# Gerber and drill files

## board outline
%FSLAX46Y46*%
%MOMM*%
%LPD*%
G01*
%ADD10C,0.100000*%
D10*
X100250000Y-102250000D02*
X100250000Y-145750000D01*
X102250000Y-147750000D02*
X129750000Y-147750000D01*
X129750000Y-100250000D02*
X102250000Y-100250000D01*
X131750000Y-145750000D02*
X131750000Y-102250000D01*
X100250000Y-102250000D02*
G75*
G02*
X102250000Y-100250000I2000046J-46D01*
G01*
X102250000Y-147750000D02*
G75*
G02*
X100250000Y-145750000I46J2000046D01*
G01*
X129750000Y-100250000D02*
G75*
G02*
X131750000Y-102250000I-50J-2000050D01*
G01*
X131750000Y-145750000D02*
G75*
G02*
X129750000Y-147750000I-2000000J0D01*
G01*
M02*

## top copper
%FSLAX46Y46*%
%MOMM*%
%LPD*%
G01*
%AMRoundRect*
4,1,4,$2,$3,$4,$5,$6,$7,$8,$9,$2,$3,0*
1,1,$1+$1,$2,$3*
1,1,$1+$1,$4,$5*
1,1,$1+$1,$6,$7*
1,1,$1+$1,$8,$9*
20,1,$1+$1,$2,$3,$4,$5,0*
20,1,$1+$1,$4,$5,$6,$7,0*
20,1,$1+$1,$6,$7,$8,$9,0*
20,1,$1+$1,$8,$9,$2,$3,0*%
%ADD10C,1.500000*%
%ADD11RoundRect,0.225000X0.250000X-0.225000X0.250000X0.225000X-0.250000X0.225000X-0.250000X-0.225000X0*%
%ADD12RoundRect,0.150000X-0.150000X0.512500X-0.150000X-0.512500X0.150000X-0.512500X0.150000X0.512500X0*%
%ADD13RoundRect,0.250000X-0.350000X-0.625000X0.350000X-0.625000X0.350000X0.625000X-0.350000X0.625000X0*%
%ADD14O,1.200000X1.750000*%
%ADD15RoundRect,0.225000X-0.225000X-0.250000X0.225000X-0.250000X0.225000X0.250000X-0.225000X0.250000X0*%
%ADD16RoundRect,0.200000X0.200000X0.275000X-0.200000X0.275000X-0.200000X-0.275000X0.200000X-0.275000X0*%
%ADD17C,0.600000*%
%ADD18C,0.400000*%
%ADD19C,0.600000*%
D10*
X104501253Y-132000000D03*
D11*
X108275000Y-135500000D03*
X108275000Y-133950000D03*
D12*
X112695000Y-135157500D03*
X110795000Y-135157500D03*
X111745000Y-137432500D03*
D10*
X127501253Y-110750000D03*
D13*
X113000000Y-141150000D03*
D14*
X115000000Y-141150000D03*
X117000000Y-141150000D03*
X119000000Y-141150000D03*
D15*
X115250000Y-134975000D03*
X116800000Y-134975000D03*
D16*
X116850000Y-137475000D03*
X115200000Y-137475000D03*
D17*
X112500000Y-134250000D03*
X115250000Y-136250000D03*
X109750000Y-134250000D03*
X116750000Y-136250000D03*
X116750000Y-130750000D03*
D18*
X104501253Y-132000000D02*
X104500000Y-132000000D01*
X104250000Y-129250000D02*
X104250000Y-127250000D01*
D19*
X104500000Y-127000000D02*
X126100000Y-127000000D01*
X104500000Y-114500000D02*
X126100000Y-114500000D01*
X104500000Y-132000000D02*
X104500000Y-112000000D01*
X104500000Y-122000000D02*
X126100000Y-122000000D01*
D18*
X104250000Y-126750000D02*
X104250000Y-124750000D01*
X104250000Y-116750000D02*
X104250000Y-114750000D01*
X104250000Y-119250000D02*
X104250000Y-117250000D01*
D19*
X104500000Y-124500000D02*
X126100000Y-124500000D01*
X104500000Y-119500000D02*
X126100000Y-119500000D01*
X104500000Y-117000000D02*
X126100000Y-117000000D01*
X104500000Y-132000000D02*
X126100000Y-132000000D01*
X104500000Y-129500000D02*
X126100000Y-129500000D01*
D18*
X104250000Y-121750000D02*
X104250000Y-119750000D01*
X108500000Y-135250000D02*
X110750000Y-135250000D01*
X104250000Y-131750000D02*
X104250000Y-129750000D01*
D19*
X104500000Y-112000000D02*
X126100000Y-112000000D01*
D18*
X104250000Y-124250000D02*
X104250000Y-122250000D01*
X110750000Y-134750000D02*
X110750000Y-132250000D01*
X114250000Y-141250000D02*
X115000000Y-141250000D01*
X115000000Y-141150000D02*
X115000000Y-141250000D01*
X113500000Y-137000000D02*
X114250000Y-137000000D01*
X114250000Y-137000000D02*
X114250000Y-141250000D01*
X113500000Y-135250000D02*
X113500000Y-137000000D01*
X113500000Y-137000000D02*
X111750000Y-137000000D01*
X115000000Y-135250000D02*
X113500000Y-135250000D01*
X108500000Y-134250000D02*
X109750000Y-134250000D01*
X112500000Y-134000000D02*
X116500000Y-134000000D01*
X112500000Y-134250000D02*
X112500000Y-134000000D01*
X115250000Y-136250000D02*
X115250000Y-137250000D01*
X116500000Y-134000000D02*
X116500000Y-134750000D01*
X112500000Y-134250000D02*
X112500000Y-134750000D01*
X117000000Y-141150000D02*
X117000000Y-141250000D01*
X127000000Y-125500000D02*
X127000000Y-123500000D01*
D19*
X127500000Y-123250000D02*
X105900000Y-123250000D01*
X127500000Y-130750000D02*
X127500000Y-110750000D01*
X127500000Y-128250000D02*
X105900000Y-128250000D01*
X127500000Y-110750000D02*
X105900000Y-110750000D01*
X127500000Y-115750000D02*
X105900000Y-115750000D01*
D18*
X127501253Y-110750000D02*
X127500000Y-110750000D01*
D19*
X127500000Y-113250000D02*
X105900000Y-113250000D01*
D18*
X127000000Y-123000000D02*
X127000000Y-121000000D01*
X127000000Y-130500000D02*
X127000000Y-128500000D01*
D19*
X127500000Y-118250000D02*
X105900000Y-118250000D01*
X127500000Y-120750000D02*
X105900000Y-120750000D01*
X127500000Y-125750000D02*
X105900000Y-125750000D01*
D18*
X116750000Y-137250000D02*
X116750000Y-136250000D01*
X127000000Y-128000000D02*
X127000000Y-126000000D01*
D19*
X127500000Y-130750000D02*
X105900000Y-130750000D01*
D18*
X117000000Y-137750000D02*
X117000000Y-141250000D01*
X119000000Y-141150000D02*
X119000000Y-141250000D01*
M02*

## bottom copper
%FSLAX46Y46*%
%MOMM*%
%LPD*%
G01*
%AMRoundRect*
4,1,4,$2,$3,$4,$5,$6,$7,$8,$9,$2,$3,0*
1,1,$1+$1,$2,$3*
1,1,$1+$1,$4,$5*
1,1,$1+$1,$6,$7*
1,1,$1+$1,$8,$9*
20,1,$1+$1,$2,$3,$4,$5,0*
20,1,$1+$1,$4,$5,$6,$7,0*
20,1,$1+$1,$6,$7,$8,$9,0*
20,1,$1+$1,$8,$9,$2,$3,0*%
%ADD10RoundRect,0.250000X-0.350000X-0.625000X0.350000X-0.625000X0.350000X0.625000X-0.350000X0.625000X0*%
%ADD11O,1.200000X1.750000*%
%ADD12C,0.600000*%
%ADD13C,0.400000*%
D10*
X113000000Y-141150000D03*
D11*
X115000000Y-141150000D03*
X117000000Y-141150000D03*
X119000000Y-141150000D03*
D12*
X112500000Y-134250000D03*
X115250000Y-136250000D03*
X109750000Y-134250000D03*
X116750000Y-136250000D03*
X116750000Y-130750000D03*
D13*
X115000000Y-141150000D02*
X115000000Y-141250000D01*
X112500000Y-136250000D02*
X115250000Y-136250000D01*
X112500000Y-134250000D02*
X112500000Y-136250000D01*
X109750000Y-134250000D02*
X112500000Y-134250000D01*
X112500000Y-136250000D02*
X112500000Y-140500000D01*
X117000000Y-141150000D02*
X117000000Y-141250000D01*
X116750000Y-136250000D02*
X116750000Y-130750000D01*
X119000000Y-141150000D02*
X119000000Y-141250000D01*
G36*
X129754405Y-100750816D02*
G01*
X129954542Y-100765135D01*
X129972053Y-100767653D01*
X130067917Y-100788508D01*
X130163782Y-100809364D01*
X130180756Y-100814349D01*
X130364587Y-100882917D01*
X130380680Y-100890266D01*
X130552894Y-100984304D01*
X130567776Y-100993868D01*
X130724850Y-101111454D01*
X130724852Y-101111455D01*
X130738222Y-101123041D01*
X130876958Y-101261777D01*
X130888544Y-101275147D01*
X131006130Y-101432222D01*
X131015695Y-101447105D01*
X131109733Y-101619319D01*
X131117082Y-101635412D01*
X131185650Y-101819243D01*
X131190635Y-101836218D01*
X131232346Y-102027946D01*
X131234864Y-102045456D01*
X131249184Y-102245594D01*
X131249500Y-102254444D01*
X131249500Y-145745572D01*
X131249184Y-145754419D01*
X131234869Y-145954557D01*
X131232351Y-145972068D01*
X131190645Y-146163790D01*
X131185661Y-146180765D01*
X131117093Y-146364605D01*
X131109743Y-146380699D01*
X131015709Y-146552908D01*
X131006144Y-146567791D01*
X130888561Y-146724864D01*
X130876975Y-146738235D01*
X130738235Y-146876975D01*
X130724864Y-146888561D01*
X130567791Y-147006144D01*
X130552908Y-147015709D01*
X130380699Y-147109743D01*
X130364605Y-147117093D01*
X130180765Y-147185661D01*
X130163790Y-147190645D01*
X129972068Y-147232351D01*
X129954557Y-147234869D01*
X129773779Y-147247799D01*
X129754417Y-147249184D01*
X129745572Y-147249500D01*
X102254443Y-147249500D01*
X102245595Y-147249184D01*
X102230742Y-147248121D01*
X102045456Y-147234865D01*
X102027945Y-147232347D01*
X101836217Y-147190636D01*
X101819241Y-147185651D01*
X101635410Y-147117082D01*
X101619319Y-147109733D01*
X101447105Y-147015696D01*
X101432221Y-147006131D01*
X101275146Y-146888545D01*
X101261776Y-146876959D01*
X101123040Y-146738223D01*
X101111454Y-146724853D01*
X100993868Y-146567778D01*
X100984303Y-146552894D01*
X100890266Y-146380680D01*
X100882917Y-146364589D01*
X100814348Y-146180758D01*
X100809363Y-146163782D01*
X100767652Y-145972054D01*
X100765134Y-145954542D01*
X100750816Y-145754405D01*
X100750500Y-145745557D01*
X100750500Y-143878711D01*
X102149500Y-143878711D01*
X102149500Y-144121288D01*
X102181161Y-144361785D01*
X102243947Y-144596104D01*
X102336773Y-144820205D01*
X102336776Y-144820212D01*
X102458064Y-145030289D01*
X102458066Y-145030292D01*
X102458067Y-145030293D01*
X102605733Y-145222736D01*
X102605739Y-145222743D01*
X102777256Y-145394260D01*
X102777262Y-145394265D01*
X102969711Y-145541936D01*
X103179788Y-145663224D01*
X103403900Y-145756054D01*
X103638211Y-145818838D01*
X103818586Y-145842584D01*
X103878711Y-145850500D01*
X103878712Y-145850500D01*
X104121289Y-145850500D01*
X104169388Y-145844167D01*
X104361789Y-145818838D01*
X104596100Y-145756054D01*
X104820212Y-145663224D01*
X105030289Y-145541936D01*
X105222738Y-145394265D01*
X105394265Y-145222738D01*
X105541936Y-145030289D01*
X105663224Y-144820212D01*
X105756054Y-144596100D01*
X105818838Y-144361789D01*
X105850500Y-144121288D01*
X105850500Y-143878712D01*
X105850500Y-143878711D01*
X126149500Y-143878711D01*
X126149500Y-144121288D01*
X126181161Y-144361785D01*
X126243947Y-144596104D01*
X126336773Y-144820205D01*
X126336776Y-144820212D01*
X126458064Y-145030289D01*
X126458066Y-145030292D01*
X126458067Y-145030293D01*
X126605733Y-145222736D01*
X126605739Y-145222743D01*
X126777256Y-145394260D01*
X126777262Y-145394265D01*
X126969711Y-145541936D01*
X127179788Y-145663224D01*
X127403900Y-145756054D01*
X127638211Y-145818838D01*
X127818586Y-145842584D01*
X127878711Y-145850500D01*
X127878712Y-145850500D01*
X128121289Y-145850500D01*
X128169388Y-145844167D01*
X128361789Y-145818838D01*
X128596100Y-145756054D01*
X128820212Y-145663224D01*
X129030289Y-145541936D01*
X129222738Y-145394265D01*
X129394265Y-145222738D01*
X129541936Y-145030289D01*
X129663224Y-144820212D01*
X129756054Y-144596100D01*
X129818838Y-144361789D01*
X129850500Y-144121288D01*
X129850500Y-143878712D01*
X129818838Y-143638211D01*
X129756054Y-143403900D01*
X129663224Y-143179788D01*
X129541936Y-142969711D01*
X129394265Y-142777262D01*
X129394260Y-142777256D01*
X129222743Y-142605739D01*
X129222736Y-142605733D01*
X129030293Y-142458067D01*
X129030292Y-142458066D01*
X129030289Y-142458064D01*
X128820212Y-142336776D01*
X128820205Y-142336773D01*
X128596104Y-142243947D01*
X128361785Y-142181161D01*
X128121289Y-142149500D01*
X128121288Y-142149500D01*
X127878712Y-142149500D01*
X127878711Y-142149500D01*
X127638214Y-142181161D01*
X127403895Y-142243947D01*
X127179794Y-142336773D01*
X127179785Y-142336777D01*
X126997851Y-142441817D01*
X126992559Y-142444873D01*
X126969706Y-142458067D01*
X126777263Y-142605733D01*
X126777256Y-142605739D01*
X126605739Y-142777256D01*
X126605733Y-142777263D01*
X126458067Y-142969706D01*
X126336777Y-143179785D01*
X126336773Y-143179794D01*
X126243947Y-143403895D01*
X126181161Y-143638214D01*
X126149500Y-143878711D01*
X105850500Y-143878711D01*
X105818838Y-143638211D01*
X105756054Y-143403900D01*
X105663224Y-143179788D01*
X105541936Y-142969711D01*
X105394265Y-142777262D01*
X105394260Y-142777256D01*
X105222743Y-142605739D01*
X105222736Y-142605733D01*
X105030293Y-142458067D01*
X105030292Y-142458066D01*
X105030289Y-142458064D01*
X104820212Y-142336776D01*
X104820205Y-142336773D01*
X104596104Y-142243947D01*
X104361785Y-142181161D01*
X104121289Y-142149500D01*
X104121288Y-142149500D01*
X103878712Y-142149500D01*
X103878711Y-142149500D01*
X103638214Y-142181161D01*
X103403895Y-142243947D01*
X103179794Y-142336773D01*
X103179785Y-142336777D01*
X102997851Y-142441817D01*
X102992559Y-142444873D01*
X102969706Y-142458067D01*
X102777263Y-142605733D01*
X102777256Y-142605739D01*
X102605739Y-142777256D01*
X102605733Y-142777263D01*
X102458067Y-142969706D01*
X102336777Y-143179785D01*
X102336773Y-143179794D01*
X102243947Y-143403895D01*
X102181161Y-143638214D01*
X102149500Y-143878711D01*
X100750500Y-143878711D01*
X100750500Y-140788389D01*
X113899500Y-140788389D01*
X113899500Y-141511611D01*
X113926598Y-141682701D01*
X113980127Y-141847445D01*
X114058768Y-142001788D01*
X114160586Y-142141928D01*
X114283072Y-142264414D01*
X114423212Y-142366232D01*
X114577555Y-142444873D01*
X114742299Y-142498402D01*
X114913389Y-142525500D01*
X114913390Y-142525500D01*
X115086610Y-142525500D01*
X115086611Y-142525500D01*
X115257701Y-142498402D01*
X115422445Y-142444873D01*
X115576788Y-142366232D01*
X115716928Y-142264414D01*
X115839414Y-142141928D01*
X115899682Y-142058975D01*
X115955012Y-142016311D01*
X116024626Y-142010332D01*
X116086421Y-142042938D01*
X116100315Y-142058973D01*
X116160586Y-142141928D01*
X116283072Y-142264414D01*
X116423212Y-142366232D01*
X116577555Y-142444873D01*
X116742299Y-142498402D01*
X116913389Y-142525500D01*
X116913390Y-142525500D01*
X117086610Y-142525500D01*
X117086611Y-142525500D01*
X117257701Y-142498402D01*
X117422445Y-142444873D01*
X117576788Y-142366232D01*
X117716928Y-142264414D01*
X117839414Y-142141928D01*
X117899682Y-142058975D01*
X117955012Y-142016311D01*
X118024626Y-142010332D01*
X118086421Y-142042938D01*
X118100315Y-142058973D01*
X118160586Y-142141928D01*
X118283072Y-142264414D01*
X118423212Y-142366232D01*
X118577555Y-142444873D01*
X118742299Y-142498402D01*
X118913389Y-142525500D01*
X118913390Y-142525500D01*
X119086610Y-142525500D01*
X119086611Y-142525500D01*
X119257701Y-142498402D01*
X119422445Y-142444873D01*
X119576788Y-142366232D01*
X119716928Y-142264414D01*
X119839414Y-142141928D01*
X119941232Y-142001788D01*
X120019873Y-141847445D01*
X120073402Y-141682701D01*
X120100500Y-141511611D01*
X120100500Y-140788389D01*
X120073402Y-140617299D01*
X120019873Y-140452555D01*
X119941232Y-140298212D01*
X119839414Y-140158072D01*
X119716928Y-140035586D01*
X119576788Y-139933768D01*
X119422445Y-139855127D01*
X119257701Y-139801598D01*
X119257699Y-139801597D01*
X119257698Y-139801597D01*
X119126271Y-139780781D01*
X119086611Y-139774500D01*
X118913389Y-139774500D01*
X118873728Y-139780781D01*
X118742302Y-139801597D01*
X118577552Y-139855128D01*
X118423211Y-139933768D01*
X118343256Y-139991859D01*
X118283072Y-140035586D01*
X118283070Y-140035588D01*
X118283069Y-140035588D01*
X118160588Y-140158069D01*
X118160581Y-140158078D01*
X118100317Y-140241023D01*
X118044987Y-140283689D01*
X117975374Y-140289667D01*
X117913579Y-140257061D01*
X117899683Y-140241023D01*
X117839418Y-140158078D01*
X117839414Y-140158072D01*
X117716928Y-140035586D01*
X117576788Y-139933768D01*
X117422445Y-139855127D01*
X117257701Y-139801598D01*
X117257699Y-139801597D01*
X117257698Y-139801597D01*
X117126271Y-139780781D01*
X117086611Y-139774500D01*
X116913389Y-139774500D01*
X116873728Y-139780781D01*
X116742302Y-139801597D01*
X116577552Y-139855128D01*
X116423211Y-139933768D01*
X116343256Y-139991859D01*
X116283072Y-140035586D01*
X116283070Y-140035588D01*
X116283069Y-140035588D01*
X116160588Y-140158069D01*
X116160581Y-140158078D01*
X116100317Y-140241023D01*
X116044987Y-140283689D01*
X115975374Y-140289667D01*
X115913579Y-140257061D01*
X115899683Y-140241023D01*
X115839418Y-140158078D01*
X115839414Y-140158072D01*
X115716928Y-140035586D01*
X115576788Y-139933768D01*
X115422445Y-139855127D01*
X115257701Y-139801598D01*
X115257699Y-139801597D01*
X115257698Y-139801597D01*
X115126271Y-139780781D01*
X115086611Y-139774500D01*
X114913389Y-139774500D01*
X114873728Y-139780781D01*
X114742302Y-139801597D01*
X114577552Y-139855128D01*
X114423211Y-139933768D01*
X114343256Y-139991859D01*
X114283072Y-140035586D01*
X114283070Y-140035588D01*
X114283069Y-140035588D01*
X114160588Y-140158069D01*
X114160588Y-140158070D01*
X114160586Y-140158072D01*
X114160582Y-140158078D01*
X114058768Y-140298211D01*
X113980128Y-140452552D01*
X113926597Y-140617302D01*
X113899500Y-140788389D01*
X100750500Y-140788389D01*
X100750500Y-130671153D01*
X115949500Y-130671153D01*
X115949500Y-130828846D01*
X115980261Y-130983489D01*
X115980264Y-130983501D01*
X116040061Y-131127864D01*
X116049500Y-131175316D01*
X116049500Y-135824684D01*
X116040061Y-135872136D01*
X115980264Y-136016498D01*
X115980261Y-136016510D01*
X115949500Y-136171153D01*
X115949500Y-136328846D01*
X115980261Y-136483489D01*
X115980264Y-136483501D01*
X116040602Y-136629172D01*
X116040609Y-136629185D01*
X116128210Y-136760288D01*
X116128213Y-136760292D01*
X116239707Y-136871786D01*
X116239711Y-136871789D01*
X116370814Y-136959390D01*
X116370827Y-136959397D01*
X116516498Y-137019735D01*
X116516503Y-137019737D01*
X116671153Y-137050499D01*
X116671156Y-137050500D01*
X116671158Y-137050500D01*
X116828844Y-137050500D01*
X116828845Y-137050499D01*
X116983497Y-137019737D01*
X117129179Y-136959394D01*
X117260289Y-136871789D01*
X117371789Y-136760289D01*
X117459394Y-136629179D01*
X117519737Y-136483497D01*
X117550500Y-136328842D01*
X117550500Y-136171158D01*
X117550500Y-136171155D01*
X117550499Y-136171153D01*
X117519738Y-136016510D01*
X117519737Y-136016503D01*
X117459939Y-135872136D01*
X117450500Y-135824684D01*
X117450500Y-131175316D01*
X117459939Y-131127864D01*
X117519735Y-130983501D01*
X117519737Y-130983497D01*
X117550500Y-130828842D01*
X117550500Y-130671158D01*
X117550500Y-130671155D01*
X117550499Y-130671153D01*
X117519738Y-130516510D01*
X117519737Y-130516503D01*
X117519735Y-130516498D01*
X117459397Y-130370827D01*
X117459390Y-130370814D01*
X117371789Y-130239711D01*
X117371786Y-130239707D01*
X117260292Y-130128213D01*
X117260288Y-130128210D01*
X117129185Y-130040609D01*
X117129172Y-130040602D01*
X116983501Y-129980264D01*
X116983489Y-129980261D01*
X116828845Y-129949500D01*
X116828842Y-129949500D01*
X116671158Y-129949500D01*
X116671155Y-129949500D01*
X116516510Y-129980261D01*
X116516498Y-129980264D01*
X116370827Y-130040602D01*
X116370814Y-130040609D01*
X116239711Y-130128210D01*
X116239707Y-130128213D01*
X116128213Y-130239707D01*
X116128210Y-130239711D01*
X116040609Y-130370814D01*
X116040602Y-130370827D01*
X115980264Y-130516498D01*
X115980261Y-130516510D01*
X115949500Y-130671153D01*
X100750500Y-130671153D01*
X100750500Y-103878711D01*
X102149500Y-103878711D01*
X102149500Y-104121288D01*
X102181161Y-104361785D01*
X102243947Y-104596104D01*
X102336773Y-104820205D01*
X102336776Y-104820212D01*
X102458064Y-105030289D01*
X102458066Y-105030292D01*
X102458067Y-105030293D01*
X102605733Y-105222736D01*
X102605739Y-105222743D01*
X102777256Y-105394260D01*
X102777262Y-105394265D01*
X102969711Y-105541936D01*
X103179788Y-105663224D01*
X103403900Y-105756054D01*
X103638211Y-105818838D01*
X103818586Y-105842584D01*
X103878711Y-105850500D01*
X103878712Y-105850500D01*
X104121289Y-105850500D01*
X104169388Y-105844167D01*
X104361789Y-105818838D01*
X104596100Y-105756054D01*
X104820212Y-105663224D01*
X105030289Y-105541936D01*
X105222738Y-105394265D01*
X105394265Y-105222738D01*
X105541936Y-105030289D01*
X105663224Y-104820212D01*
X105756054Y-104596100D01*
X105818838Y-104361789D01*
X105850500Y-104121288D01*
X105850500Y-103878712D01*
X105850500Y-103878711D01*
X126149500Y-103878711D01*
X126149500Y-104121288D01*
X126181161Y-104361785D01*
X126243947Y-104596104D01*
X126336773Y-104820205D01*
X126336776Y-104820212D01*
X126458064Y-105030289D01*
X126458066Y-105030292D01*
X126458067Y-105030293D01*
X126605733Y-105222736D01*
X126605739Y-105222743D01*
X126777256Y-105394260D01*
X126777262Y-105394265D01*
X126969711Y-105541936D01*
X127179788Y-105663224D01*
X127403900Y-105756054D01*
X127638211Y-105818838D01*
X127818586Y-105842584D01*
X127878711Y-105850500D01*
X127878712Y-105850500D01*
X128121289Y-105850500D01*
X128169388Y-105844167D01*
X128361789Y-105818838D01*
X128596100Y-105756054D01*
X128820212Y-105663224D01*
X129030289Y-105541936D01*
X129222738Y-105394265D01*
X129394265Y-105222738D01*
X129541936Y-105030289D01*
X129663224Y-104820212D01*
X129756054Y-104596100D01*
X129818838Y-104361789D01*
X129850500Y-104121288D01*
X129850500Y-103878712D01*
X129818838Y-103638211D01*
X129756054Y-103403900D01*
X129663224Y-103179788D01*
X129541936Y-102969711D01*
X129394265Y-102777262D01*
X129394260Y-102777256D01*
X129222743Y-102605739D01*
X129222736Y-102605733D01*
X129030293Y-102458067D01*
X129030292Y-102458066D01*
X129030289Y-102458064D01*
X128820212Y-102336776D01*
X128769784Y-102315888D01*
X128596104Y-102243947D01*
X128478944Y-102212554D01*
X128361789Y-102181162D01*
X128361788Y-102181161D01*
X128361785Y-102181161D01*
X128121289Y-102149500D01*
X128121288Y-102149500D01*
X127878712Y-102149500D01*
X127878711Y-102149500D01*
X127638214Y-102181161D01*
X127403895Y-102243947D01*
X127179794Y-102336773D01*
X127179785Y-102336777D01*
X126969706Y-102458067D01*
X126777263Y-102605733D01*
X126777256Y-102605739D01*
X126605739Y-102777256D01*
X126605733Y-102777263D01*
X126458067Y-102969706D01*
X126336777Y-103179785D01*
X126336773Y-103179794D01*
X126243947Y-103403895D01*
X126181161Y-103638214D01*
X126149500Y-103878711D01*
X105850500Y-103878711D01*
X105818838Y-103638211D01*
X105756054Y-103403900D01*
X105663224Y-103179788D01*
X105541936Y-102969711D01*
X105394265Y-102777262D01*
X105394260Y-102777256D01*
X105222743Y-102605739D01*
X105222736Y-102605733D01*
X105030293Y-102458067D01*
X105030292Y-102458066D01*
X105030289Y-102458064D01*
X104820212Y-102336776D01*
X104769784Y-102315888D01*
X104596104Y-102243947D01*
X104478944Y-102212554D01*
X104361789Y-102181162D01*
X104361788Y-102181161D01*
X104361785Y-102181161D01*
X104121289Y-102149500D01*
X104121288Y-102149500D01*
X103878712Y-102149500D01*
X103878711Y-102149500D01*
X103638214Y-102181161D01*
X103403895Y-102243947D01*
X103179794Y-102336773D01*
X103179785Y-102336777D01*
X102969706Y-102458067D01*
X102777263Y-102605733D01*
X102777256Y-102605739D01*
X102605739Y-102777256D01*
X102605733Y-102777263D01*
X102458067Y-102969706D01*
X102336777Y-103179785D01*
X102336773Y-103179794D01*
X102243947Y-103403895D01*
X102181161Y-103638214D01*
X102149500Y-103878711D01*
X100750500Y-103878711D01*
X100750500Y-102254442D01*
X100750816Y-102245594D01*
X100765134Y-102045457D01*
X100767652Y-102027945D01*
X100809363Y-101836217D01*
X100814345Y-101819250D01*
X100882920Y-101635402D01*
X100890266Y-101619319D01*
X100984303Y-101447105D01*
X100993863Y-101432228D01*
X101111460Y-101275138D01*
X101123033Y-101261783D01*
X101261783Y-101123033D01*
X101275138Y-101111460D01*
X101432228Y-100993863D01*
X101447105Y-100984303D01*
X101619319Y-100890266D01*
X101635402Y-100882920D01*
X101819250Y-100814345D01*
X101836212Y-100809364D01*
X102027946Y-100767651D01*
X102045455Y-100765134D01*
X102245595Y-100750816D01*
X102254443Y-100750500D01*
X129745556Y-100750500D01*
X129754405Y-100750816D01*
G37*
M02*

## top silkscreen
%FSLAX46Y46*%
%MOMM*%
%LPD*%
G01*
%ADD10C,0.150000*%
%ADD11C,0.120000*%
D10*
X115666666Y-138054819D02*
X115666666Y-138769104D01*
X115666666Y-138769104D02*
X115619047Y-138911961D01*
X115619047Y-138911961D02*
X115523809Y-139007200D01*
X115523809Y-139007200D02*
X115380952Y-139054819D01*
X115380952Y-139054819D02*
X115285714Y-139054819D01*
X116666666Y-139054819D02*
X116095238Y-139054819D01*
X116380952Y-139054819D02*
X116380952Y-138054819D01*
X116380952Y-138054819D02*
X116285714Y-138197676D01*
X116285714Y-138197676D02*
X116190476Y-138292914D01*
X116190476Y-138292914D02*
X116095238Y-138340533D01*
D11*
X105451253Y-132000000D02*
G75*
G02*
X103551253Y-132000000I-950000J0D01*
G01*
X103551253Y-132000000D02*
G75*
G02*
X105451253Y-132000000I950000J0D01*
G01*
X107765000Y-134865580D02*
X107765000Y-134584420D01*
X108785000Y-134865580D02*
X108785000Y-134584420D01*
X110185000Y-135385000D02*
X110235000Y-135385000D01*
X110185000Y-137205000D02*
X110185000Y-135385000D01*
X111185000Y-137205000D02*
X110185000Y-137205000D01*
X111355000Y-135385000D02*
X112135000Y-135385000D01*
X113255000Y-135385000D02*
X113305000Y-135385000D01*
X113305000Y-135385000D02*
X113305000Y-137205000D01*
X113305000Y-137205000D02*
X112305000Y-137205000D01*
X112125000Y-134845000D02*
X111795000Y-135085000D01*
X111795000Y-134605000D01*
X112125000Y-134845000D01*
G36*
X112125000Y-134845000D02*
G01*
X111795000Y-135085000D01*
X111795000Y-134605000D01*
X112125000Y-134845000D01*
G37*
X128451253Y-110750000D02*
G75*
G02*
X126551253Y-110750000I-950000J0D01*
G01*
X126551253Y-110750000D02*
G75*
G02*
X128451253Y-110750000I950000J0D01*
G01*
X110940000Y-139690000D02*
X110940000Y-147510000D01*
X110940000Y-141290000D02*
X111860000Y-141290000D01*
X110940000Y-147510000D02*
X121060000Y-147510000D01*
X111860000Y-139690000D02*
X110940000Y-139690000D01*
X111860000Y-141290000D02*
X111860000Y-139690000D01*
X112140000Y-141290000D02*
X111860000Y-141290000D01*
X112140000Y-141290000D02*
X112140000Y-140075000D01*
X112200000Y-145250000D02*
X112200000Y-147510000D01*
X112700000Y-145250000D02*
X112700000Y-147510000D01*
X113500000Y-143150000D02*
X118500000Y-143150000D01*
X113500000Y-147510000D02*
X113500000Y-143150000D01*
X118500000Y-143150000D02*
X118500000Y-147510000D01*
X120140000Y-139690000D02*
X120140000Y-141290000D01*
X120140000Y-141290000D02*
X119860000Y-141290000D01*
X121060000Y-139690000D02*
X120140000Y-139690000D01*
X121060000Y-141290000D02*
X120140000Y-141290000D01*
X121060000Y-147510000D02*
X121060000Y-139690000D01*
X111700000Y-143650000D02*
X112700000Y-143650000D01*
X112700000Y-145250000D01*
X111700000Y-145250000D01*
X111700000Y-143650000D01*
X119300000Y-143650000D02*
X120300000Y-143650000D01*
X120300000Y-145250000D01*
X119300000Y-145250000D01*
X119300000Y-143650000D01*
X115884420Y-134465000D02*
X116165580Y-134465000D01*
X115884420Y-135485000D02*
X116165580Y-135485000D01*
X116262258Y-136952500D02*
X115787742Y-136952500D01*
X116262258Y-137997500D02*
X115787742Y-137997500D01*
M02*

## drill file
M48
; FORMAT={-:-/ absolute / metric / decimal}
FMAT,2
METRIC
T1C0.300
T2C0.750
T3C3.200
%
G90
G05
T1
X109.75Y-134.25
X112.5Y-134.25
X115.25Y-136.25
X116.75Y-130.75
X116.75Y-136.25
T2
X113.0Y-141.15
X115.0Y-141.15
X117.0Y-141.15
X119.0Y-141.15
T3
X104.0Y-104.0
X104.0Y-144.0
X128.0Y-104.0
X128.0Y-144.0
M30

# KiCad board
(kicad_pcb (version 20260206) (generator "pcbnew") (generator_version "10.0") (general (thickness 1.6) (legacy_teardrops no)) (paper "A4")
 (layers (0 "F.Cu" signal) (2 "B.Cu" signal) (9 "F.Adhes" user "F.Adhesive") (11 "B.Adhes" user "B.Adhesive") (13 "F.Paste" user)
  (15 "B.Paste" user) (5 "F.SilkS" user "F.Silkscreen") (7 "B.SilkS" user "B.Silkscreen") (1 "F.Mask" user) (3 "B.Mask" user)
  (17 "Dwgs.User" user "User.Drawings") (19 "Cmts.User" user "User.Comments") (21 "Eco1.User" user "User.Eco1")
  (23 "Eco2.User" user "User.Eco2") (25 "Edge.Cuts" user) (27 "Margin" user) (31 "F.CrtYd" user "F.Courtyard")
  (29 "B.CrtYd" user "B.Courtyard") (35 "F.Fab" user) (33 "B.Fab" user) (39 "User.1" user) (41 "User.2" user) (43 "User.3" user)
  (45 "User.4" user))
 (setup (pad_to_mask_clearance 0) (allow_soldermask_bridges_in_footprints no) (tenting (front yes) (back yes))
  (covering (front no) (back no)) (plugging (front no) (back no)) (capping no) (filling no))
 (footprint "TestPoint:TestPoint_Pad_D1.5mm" (layer "F.Cu") (at 104.501253 132)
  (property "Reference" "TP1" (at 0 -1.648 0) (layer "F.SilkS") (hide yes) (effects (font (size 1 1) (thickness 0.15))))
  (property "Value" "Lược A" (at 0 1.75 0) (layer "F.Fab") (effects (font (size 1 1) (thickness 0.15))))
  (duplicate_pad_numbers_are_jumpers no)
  (fp_circle (center 0 0) (end 0 0.95) (stroke (width 0.12) (type solid)) (fill no) (layer "F.SilkS"))
  (pad "1" smd circle (at 0 0) (size 1.5 1.5) (layers "F.Cu" "F.Mask") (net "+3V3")))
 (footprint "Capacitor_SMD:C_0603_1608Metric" (layer "F.Cu") (at 108.275 134.725 90)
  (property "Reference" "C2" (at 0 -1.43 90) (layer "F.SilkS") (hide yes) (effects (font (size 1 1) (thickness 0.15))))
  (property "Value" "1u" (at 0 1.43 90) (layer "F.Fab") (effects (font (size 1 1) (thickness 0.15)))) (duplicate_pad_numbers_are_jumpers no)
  (fp_line (start -0.14058 -0.51) (end 0.14058 -0.51) (stroke (width 0.12) (type solid)) (layer "F.SilkS"))
  (fp_line (start -0.14058 0.51) (end 0.14058 0.51) (stroke (width 0.12) (type solid)) (layer "F.SilkS"))
  (pad "1" smd roundrect (at -0.775 0 90) (size 0.9 0.95) (layers "F.Cu" "F.Mask" "F.Paste") (roundrect_rratio 0.25) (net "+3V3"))
  (pad "2" smd roundrect (at 0.775 0 90) (size 0.9 0.95) (layers "F.Cu" "F.Mask" "F.Paste") (roundrect_rratio 0.25) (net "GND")))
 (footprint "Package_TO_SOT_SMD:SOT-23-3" (layer "F.Cu") (at 111.745 136.295 -90)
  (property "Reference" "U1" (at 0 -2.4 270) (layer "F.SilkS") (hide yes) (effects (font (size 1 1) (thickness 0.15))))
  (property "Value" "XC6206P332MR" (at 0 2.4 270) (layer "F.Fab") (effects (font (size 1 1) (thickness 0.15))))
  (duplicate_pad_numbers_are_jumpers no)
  (fp_line (start -0.91 1.56) (end -0.91 1.51) (stroke (width 0.12) (type solid)) (layer "F.SilkS"))
  (fp_line (start 0.91 1.56) (end -0.91 1.56) (stroke (width 0.12) (type solid)) (layer "F.SilkS"))
  (fp_line (start 0.91 0.56) (end 0.91 1.56) (stroke (width 0.12) (type solid)) (layer "F.SilkS"))
  (fp_line (start -0.91 0.39) (end -0.91 -0.39) (stroke (width 0.12) (type solid)) (layer "F.SilkS"))
  (fp_line (start -0.91 -1.51) (end -0.91 -1.56) (stroke (width 0.12) (type solid)) (layer "F.SilkS"))
  (fp_line (start -0.91 -1.56) (end 0.91 -1.56) (stroke (width 0.12) (type solid)) (layer "F.SilkS"))
  (fp_line (start 0.91 -1.56) (end 0.91 -0.56) (stroke (width 0.12) (type solid)) (layer "F.SilkS"))
  (fp_poly (pts (xy -1.45 -0.38) (xy -1.21 -0.05) (xy -1.69 -0.05)) (stroke (width 0.12) (type solid)) (fill yes) (layer "F.SilkS"))
  (pad "1" smd roundrect (at -1.1375 -0.95 270) (size 1.325 0.6) (layers "F.Cu" "F.Mask" "F.Paste") (roundrect_rratio 0.25) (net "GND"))
  (pad "2" smd roundrect (at -1.1375 0.95 270) (size 1.325 0.6) (layers "F.Cu" "F.Mask" "F.Paste") (roundrect_rratio 0.25) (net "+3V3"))
  (pad "3" smd roundrect (at 1.1375 0 270) (size 1.325 0.6) (layers "F.Cu" "F.Mask" "F.Paste") (roundrect_rratio 0.25) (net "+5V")))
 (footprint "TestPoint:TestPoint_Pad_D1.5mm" (layer "F.Cu") (at 127.501253 110.75)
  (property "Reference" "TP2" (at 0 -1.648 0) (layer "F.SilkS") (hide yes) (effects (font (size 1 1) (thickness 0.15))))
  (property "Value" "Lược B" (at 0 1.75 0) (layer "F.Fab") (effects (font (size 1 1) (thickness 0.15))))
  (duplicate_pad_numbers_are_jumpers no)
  (fp_circle (center 0 0) (end 0 0.95) (stroke (width 0.12) (type solid)) (fill no) (layer "F.SilkS"))
  (pad "1" smd circle (at 0 0) (size 1.5 1.5) (layers "F.Cu" "F.Mask") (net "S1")))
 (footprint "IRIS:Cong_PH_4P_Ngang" (layer "F.Cu") (at 113 141.15)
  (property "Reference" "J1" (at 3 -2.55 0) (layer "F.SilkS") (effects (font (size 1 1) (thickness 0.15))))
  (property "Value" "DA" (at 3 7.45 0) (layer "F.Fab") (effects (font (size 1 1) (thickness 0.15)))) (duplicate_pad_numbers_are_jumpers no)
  (fp_line (start -2.06 -1.46) (end -2.06 6.36) (stroke (width 0.12) (type solid)) (layer "F.SilkS"))
  (fp_line (start -2.06 0.14) (end -1.14 0.14) (stroke (width 0.12) (type solid)) (layer "F.SilkS"))
  (fp_line (start -2.06 6.36) (end 8.06 6.36) (stroke (width 0.12) (type solid)) (layer "F.SilkS"))
  (fp_line (start -1.14 -1.46) (end -2.06 -1.46) (stroke (width 0.12) (type solid)) (layer "F.SilkS"))
  (fp_line (start -1.14 0.14) (end -1.14 -1.46) (stroke (width 0.12) (type solid)) (layer "F.SilkS"))
  (fp_line (start -0.86 0.14) (end -1.14 0.14) (stroke (width 0.12) (type solid)) (layer "F.SilkS"))
  (fp_line (start -0.86 0.14) (end -0.86 -1.075) (stroke (width 0.12) (type solid)) (layer "F.SilkS"))
  (fp_line (start -0.8 4.1) (end -0.8 6.36) (stroke (width 0.12) (type solid)) (layer "F.SilkS"))
  (fp_line (start -0.3 4.1) (end -0.3 6.36) (stroke (width 0.12) (type solid)) (layer "F.SilkS"))
  (fp_line (start 0.5 2) (end 5.5 2) (stroke (width 0.12) (type solid)) (layer "F.SilkS"))
  (fp_line (start 0.5 6.36) (end 0.5 2) (stroke (width 0.12) (type solid)) (layer "F.SilkS"))
  (fp_line (start 5.5 2) (end 5.5 6.36) (stroke (width 0.12) (type solid)) (layer "F.SilkS"))
  (fp_line (start 7.14 -1.46) (end 7.14 0.14) (stroke (width 0.12) (type solid)) (layer "F.SilkS"))
  (fp_line (start 7.14 0.14) (end 6.86 0.14) (stroke (width 0.12) (type solid)) (layer "F.SilkS"))
  (fp_line (start 8.06 -1.46) (end 7.14 -1.46) (stroke (width 0.12) (type solid)) (layer "F.SilkS"))
  (fp_line (start 8.06 0.14) (end 7.14 0.14) (stroke (width 0.12) (type solid)) (layer "F.SilkS"))
  (fp_line (start 8.06 6.36) (end 8.06 -1.46) (stroke (width 0.12) (type solid)) (layer "F.SilkS"))
  (fp_rect (start -1.3 2.5) (end -0.3 4.1) (stroke (width 0.12) (type solid)) (fill no) (layer "F.SilkS"))
  (fp_rect (start 6.3 2.5) (end 7.3 4.1) (stroke (width 0.12) (type solid)) (fill no) (layer "F.SilkS"))
  (pad "1" thru_hole roundrect (at 0 0) (size 1.2 1.75) (drill 0.75) (layers "*.Cu" "*.Mask") (remove_unused_layers no)
   (roundrect_rratio 0.208333) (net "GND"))
  (pad "2" thru_hole oval (at 2 0) (size 1.2 1.75) (drill 0.75) (layers "*.Cu" "*.Mask") (remove_unused_layers no) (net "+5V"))
  (pad "3" thru_hole oval (at 4 0) (size 1.2 1.75) (drill 0.75) (layers "*.Cu" "*.Mask") (remove_unused_layers no) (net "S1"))
  (pad "4" thru_hole oval (at 6 0) (size 1.2 1.75) (drill 0.75) (layers "*.Cu" "*.Mask") (remove_unused_layers no)
   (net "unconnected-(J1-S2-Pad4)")))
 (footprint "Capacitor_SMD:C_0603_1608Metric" (layer "F.Cu") (at 116.025 134.975)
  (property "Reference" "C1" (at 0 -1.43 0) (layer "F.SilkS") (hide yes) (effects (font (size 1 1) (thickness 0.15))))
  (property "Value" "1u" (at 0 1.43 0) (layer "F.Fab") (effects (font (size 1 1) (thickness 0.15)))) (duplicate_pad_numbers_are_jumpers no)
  (fp_line (start -0.14058 -0.51) (end 0.14058 -0.51) (stroke (width 0.12) (type solid)) (layer "F.SilkS"))
  (fp_line (start -0.14058 0.51) (end 0.14058 0.51) (stroke (width 0.12) (type solid)) (layer "F.SilkS"))
  (pad "1" smd roundrect (at -0.775 0) (size 0.9 0.95) (layers "F.Cu" "F.Mask" "F.Paste") (roundrect_rratio 0.25) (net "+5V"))
  (pad "2" smd roundrect (at 0.775 0) (size 0.9 0.95) (layers "F.Cu" "F.Mask" "F.Paste") (roundrect_rratio 0.25) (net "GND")))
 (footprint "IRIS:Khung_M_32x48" (layer "F.Cu") (at 100 148)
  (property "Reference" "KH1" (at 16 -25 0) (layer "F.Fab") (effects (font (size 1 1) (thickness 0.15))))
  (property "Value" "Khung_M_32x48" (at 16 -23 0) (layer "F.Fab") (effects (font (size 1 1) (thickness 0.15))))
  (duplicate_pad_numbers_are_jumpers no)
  (fp_line (start 0.25 -45.75) (end 0.25 -2.25) (stroke (width 0.1) (type solid)) (layer "Edge.Cuts"))
  (fp_line (start 2.25 -0.25) (end 29.75 -0.25) (stroke (width 0.1) (type solid)) (layer "Edge.Cuts"))
  (fp_line (start 29.75 -47.75) (end 2.25 -47.75) (stroke (width 0.1) (type solid)) (layer "Edge.Cuts"))
  (fp_line (start 31.75 -2.25) (end 31.75 -45.75) (stroke (width 0.1) (type solid)) (layer "Edge.Cuts"))
  (fp_arc (start 0.25 -45.75) (mid 0.8358 -47.1642) (end 2.25 -47.75) (stroke (width 0.1) (type solid)) (layer "Edge.Cuts"))
  (fp_arc (start 2.25 -0.25) (mid 0.8358 -0.8358) (end 0.25 -2.25) (stroke (width 0.1) (type solid)) (layer "Edge.Cuts"))
  (fp_arc (start 29.75 -47.75) (mid 31.164199 -47.164199) (end 31.75 -45.75) (stroke (width 0.1) (type solid)) (layer "Edge.Cuts"))
  (fp_arc (start 31.75 -2.25) (mid 31.164214 -0.835786) (end 29.75 -0.25) (stroke (width 0.1) (type solid)) (layer "Edge.Cuts"))
  (pad "" np_thru_hole circle (at 4 -44) (size 3.2 3.2) (drill 3.2) (layers "*.Cu" "*.Mask"))
  (pad "" np_thru_hole circle (at 4 -4) (size 3.2 3.2) (drill 3.2) (layers "*.Cu" "*.Mask"))
  (pad "" np_thru_hole circle (at 28 -44) (size 3.2 3.2) (drill 3.2) (layers "*.Cu" "*.Mask"))
  (pad "" np_thru_hole circle (at 28 -4) (size 3.2 3.2) (drill 3.2) (layers "*.Cu" "*.Mask")))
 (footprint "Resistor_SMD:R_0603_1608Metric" (layer "F.Cu") (at 116.025 137.475 180)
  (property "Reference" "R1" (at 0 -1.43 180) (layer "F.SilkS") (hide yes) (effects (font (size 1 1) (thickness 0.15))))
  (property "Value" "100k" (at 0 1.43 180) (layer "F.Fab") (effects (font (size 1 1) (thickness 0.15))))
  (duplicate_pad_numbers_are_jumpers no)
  (fp_line (start -0.237258 0.5225) (end 0.237258 0.5225) (stroke (width 0.12) (type solid)) (layer "F.SilkS"))
  (fp_line (start -0.237258 -0.5225) (end 0.237258 -0.5225) (stroke (width 0.12) (type solid)) (layer "F.SilkS"))
  (pad "1" smd roundrect (at -0.825 0 180) (size 0.8 0.95) (layers "F.Cu" "F.Mask" "F.Paste") (roundrect_rratio 0.25) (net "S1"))
  (pad "2" smd roundrect (at 0.825 0 180) (size 0.8 0.95) (layers "F.Cu" "F.Mask" "F.Paste") (roundrect_rratio 0.25) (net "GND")))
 (segment (start 104.501253 132) (end 104.5 132) (width 0.4) (layer "F.Cu") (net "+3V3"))
 (segment (start 104.25 129.25) (end 104.25 127.25) (width 0.4) (layer "F.Cu") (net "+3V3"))
 (segment (start 104.5 127) (end 126.1 127) (width 0.6) (layers "F.Cu" "F.Mask") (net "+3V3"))
 (segment (start 104.5 114.5) (end 126.1 114.5) (width 0.6) (layers "F.Cu" "F.Mask") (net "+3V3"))
 (segment (start 104.5 132) (end 104.5 112) (width 0.6) (layers "F.Cu" "F.Mask") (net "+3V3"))
 (segment (start 104.5 122) (end 126.1 122) (width 0.6) (layers "F.Cu" "F.Mask") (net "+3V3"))
 (segment (start 104.25 126.75) (end 104.25 124.75) (width 0.4) (layer "F.Cu") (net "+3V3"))
 (segment (start 104.25 116.75) (end 104.25 114.75) (width 0.4) (layer "F.Cu") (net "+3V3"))
 (segment (start 104.25 119.25) (end 104.25 117.25) (width 0.4) (layer "F.Cu") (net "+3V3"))
 (segment (start 104.5 124.5) (end 126.1 124.5) (width 0.6) (layers "F.Cu" "F.Mask") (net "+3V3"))
 (segment (start 104.5 119.5) (end 126.1 119.5) (width 0.6) (layers "F.Cu" "F.Mask") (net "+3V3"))
 (segment (start 104.5 117) (end 126.1 117) (width 0.6) (layers "F.Cu" "F.Mask") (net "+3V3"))
 (segment (start 104.5 132) (end 126.1 132) (width 0.6) (layers "F.Cu" "F.Mask") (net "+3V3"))
 (segment (start 104.5 129.5) (end 126.1 129.5) (width 0.6) (layers "F.Cu" "F.Mask") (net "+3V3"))
 (segment (start 104.25 121.75) (end 104.25 119.75) (width 0.4) (layer "F.Cu") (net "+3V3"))
 (segment (start 108.5 135.25) (end 110.75 135.25) (width 0.4) (layer "F.Cu") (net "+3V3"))
 (segment (start 104.25 131.75) (end 104.25 129.75) (width 0.4) (layer "F.Cu") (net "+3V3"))
 (segment (start 104.5 112) (end 126.1 112) (width 0.6) (layers "F.Cu" "F.Mask") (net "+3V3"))
 (segment (start 104.25 124.25) (end 104.25 122.25) (width 0.4) (layer "F.Cu") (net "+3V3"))
 (segment (start 110.75 134.75) (end 110.75 132.25) (width 0.4) (layer "F.Cu") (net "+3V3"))
 (segment (start 114.25 141.25) (end 115 141.25) (width 0.4) (layer "F.Cu") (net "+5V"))
 (segment (start 115 141.15) (end 115 141.25) (width 0.4) (layer "F.Cu") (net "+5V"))
 (segment (start 113.5 137) (end 114.25 137) (width 0.4) (layer "F.Cu") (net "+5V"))
 (segment (start 114.25 137) (end 114.25 141.25) (width 0.4) (layer "F.Cu") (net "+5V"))
 (segment (start 113.5 135.25) (end 113.5 137) (width 0.4) (layer "F.Cu") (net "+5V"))
 (segment (start 113.5 137) (end 111.75 137) (width 0.4) (layer "F.Cu") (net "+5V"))
 (segment (start 115 135.25) (end 113.5 135.25) (width 0.4) (layer "F.Cu") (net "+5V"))
 (segment (start 115 141.15) (end 115 141.25) (width 0.4) (layer "B.Cu") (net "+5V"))
 (segment (start 108.5 134.25) (end 109.75 134.25) (width 0.4) (layer "F.Cu") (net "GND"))
 (segment (start 112.5 134) (end 116.5 134) (width 0.4) (layer "F.Cu") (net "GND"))
 (segment (start 112.5 134.25) (end 112.5 134) (width 0.4) (layer "F.Cu") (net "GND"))
 (segment (start 115.25 136.25) (end 115.25 137.25) (width 0.4) (layer "F.Cu") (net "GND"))
 (segment (start 116.5 134) (end 116.5 134.75) (width 0.4) (layer "F.Cu") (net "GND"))
 (segment (start 112.5 134.25) (end 112.5 134.75) (width 0.4) (layer "F.Cu") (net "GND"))
 (via (at 112.5 134.25) (size 0.6) (drill 0.3) (layers "F.Cu" "B.Cu") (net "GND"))
 (via (at 115.25 136.25) (size 0.6) (drill 0.3) (layers "F.Cu" "B.Cu") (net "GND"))
 (via (at 109.75 134.25) (size 0.6) (drill 0.3) (layers "F.Cu" "B.Cu") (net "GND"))
 (segment (start 112.5 136.25) (end 115.25 136.25) (width 0.4) (layer "B.Cu") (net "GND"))
 (segment (start 112.5 134.25) (end 112.5 136.25) (width 0.4) (layer "B.Cu") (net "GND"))
 (segment (start 109.75 134.25) (end 112.5 134.25) (width 0.4) (layer "B.Cu") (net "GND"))
 (segment (start 112.5 136.25) (end 112.5 140.5) (width 0.4) (layer "B.Cu") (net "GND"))
 (segment (start 117 141.15) (end 117 141.25) (width 0.4) (layer "F.Cu") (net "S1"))
 (segment (start 127 125.5) (end 127 123.5) (width 0.4) (layer "F.Cu") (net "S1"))
 (segment (start 127.5 123.25) (end 105.9 123.25) (width 0.6) (layers "F.Cu" "F.Mask") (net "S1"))
 (segment (start 127.5 130.75) (end 127.5 110.75) (width 0.6) (layers "F.Cu" "F.Mask") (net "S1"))
 (segment (start 127.5 128.25) (end 105.9 128.25) (width 0.6) (layers "F.Cu" "F.Mask") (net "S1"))
 (segment (start 127.5 110.75) (end 105.9 110.75) (width 0.6) (layers "F.Cu" "F.Mask") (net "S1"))
 (segment (start 127.5 115.75) (end 105.9 115.75) (width 0.6) (layers "F.Cu" "F.Mask") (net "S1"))
 (segment (start 127.501253 110.75) (end 127.5 110.75) (width 0.4) (layer "F.Cu") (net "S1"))
 (segment (start 127.5 113.25) (end 105.9 113.25) (width 0.6) (layers "F.Cu" "F.Mask") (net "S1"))
 (segment (start 127 123) (end 127 121) (width 0.4) (layer "F.Cu") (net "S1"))
 (segment (start 127 130.5) (end 127 128.5) (width 0.4) (layer "F.Cu") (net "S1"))
 (segment (start 127.5 118.25) (end 105.9 118.25) (width 0.6) (layers "F.Cu" "F.Mask") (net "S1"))
 (segment (start 127.5 120.75) (end 105.9 120.75) (width 0.6) (layers "F.Cu" "F.Mask") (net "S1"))
 (segment (start 127.5 125.75) (end 105.9 125.75) (width 0.6) (layers "F.Cu" "F.Mask") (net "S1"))
 (segment (start 116.75 137.25) (end 116.75 136.25) (width 0.4) (layer "F.Cu") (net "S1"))
 (segment (start 127 128) (end 127 126) (width 0.4) (layer "F.Cu") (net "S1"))
 (segment (start 127.5 130.75) (end 105.9 130.75) (width 0.6) (layers "F.Cu" "F.Mask") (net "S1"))
 (segment (start 117 137.75) (end 117 141.25) (width 0.4) (layer "F.Cu") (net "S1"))
 (via (at 116.75 136.25) (size 0.6) (drill 0.3) (layers "F.Cu" "B.Cu") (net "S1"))
 (via (at 116.75 130.75) (size 0.6) (drill 0.3) (layers "F.Cu" "B.Cu") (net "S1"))
 (segment (start 117 141.15) (end 117 141.25) (width 0.4) (layer "B.Cu") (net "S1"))
 (segment (start 116.75 136.25) (end 116.75 130.75) (width 0.4) (layer "B.Cu") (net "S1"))
 (segment (start 119 141.15) (end 119 141.25) (width 0.4) (layer "F.Cu") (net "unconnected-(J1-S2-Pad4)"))
 (segment (start 119 141.15) (end 119 141.25) (width 0.4) (layer "B.Cu") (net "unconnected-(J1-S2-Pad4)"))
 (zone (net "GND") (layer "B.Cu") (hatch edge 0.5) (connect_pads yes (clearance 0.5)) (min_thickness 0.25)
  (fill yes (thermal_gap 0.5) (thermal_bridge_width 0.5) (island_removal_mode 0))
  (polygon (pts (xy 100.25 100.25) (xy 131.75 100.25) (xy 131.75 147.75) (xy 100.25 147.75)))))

